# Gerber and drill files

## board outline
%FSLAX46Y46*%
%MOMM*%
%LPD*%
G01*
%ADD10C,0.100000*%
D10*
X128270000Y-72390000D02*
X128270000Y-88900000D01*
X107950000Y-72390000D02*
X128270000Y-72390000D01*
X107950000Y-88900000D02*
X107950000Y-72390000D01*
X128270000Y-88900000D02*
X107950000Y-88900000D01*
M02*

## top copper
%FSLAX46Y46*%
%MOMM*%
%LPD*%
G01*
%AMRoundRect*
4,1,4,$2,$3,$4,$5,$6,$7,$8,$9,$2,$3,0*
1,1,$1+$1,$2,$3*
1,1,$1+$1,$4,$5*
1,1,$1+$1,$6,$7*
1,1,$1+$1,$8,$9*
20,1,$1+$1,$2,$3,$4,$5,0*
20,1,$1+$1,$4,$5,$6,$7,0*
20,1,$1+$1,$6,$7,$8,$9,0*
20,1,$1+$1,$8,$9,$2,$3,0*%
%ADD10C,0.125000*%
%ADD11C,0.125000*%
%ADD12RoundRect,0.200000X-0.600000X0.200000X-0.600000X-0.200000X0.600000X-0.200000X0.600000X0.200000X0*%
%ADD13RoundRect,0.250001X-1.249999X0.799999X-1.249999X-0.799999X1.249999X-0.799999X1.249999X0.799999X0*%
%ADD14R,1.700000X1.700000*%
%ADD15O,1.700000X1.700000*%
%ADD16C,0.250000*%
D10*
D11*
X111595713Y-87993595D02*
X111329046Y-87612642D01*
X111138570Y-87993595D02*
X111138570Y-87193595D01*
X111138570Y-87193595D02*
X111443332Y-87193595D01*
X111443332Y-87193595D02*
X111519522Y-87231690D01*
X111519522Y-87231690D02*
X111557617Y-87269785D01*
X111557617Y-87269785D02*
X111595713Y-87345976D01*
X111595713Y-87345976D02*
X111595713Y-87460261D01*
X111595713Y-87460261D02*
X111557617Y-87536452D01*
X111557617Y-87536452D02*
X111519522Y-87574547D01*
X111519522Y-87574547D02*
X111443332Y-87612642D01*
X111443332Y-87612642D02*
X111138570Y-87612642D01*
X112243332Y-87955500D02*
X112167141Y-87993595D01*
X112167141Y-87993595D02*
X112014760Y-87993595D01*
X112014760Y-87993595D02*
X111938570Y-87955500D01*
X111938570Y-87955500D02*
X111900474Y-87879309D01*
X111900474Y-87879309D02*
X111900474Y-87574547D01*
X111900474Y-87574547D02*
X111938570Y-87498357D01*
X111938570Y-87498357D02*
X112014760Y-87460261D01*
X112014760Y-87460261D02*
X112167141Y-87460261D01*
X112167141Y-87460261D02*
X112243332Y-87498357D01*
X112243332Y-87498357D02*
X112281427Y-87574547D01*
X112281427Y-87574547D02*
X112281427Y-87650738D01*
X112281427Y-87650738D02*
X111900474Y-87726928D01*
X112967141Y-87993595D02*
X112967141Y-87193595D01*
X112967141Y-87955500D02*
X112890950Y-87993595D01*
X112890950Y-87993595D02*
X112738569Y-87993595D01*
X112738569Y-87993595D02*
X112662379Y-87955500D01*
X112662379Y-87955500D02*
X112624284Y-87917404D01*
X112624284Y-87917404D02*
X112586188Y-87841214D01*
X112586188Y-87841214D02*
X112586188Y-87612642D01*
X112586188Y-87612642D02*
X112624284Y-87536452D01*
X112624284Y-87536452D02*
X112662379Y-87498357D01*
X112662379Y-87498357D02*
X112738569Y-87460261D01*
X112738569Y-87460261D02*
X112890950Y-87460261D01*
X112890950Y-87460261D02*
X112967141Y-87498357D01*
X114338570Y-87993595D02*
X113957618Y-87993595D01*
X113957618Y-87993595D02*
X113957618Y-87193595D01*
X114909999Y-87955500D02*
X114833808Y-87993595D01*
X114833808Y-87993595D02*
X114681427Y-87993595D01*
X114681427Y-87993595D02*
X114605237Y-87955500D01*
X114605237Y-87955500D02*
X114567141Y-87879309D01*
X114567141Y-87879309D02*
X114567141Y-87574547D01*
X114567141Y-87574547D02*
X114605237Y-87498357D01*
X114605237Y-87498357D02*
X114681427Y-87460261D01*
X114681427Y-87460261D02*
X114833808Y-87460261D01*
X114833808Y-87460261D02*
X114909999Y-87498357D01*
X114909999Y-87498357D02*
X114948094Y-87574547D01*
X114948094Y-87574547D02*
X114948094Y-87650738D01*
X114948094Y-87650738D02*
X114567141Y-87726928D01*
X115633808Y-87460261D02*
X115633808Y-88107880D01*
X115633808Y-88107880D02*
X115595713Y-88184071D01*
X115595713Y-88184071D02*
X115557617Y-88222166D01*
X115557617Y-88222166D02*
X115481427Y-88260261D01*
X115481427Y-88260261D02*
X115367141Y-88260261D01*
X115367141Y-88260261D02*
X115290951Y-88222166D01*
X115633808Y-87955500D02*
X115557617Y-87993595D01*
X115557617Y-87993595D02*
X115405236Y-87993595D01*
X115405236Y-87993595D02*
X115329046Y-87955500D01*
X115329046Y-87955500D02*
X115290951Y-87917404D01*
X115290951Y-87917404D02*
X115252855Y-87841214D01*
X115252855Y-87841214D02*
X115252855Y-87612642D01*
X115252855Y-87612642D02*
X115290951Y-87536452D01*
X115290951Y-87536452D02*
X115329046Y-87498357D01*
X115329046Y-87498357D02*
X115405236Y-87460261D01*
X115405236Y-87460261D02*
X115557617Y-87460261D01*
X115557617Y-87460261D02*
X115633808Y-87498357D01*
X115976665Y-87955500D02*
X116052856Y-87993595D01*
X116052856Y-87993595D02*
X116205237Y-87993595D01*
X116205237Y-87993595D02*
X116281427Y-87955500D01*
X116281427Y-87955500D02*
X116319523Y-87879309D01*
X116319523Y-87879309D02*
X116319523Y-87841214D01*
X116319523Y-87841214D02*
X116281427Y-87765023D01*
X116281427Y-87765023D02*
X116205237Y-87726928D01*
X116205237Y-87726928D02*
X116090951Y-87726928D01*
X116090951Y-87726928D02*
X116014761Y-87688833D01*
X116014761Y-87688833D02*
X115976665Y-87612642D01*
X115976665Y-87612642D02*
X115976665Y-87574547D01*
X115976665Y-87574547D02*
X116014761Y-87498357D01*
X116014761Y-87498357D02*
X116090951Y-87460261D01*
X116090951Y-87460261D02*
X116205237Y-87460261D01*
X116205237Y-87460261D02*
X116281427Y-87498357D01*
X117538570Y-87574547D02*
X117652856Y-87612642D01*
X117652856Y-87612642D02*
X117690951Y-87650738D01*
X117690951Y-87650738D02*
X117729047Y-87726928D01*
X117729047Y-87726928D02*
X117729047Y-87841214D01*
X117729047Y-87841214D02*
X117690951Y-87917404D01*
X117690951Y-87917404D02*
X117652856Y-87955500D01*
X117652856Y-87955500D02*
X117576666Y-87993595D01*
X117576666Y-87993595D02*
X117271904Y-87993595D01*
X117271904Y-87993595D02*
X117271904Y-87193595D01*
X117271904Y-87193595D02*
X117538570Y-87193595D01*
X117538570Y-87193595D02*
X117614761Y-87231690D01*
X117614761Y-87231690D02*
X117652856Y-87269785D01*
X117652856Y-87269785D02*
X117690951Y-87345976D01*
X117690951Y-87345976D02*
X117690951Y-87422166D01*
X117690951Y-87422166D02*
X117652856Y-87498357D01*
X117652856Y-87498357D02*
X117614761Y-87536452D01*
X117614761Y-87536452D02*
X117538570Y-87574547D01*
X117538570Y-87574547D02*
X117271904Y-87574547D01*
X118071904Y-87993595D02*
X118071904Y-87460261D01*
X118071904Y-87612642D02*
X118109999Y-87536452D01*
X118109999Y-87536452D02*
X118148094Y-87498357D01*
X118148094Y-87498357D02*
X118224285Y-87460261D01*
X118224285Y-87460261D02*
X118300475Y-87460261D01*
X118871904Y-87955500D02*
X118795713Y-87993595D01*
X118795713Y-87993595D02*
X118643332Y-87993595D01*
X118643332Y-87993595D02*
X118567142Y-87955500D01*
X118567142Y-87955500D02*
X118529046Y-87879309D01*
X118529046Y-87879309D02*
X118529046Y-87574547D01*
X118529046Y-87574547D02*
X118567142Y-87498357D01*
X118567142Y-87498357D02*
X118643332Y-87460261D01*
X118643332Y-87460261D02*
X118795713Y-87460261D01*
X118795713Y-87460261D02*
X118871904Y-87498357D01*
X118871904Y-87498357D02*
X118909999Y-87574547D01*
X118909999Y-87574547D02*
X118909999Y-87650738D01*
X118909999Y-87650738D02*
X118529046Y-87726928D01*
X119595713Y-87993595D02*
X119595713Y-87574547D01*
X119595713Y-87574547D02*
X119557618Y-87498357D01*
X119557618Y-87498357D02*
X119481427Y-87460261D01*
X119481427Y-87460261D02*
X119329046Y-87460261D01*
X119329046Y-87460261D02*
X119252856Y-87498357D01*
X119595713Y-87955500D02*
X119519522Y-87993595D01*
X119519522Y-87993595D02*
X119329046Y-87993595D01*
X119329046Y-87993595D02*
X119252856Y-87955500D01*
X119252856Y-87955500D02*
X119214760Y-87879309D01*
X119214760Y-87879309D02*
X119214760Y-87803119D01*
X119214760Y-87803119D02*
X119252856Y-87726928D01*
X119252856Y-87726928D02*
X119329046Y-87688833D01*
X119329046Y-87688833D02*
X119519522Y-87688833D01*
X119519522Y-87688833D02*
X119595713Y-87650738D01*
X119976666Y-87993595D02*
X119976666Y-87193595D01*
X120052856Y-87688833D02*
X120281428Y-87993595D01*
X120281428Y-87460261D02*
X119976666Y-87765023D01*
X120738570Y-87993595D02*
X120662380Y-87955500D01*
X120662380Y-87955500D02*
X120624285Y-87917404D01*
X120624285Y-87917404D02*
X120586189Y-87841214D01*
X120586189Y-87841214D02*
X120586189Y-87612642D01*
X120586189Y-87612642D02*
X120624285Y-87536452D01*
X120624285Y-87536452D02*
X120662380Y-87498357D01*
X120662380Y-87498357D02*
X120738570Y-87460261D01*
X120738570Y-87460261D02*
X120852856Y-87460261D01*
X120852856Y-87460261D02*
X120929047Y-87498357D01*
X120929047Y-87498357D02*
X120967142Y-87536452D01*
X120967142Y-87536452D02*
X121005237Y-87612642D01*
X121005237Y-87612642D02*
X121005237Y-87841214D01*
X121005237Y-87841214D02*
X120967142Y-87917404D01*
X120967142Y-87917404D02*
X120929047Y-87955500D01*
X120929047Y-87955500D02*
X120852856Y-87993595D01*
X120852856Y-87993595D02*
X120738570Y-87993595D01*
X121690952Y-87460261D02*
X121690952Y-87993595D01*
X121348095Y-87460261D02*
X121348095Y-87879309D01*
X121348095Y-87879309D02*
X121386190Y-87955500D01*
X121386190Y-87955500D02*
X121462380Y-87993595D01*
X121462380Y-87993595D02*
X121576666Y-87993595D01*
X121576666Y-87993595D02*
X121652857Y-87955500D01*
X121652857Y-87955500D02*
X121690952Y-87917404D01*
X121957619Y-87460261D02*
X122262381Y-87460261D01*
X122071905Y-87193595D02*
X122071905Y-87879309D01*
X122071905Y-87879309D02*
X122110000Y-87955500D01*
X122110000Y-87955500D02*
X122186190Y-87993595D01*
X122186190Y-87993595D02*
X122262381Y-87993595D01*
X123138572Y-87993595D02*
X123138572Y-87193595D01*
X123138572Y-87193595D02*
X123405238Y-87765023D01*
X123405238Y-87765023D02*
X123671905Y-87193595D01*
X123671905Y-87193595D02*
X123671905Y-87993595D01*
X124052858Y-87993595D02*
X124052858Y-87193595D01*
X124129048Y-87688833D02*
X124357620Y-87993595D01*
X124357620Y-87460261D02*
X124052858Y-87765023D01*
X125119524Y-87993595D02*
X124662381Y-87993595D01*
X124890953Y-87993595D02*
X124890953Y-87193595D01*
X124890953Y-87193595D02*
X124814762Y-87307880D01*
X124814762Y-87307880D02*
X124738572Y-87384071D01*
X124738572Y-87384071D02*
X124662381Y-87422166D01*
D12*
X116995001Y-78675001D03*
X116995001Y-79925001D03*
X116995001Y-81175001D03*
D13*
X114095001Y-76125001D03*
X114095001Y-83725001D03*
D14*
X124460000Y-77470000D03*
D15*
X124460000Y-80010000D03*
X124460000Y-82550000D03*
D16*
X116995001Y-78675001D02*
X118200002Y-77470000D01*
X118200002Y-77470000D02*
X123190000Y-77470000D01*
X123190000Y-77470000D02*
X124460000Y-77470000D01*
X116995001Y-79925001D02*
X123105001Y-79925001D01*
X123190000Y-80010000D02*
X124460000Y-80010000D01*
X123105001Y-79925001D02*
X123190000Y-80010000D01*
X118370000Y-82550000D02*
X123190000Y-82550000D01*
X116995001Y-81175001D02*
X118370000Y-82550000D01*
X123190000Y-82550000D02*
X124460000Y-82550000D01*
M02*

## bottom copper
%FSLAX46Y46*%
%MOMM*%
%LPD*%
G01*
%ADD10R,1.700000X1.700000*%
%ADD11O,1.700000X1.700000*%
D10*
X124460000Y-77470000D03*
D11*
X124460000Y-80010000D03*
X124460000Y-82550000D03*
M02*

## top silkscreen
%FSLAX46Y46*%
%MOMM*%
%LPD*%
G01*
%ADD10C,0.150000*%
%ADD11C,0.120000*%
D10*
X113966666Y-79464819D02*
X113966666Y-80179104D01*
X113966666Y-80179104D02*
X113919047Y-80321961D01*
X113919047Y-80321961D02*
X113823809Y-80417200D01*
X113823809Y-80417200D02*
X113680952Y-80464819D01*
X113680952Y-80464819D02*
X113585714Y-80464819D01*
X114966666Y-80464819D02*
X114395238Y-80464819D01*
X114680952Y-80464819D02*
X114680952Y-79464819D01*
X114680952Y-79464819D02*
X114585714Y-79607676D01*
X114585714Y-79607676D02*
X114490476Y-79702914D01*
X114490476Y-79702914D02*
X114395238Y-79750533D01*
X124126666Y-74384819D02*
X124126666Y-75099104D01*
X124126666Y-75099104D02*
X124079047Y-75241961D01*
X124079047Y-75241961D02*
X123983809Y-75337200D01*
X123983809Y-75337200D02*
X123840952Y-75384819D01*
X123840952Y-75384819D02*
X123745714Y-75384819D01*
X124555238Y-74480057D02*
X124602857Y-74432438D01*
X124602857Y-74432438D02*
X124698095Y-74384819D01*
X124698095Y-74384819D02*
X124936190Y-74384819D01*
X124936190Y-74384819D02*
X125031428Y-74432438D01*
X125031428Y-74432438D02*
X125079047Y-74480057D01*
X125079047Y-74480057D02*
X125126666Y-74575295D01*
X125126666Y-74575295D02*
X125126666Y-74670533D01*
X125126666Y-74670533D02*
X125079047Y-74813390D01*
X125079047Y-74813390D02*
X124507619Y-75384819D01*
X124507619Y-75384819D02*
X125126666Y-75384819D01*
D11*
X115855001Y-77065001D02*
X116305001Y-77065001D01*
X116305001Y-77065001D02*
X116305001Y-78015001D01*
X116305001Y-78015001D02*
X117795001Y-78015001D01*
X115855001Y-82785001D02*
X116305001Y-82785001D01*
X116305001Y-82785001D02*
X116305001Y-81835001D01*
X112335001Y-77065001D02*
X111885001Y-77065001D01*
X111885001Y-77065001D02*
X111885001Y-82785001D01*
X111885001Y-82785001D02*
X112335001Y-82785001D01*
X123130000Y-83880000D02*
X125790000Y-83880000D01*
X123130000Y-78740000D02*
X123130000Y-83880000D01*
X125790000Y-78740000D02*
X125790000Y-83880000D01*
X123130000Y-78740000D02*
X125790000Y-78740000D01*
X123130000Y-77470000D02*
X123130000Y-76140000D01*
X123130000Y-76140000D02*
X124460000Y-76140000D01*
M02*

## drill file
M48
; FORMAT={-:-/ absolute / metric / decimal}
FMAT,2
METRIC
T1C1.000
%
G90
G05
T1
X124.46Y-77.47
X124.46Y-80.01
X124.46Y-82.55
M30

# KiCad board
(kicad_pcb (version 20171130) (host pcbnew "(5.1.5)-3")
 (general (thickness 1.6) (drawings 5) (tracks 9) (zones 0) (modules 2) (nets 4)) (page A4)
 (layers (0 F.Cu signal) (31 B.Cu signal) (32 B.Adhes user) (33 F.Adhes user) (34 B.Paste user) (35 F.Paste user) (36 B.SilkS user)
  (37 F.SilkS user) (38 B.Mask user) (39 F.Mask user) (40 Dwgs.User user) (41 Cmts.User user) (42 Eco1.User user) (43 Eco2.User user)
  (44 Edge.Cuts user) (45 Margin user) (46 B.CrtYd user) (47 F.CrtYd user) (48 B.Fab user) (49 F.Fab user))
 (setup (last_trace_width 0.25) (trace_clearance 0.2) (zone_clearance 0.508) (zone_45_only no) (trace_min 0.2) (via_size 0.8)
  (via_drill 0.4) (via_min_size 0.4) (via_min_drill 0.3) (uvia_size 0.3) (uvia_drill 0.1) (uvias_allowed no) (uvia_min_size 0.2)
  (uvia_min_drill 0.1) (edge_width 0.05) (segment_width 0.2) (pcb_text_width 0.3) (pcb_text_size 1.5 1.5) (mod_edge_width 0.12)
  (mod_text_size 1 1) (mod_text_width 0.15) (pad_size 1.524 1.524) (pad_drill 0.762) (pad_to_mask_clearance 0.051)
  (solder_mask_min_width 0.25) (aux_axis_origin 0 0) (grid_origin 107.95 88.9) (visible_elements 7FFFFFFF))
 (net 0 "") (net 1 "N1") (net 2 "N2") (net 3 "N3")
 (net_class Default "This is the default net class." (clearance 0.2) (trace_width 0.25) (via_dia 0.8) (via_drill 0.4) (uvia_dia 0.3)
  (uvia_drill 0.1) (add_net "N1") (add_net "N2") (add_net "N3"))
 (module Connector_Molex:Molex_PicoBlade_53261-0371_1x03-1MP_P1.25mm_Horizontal (layer F.Cu) (at 114.595001 79.925001 270)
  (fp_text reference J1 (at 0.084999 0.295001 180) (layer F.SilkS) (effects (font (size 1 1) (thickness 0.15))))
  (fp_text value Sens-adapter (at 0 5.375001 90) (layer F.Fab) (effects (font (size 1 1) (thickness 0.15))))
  (fp_line (start -2.86 -1.26) (end -2.86 -1.71) (layer F.SilkS) (width 0.12))
  (fp_line (start -2.86 -1.71) (end -1.91 -1.71) (layer F.SilkS) (width 0.12))
  (fp_line (start -1.91 -1.71) (end -1.91 -3.2) (layer F.SilkS) (width 0.12))
  (fp_line (start 2.86 -1.26) (end 2.86 -1.71) (layer F.SilkS) (width 0.12))
  (fp_line (start 2.86 -1.71) (end 1.91 -1.71) (layer F.SilkS) (width 0.12))
  (fp_line (start -2.86 2.26) (end -2.86 2.71) (layer F.SilkS) (width 0.12))
  (fp_line (start -2.86 2.71) (end 2.86 2.71) (layer F.SilkS) (width 0.12))
  (fp_line (start 2.86 2.71) (end 2.86 2.26) (layer F.SilkS) (width 0.12))
  (pad 1 smd roundrect (at -1.25 -2.4 270) (size 0.8 1.6) (layers F.Cu F.Paste F.Mask) (roundrect_rratio 0.25) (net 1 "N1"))
  (pad 2 smd roundrect (at 0 -2.4 270) (size 0.8 1.6) (layers F.Cu F.Paste F.Mask) (roundrect_rratio 0.25) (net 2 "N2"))
  (pad 3 smd roundrect (at 1.25 -2.4 270) (size 0.8 1.6) (layers F.Cu F.Paste F.Mask) (roundrect_rratio 0.25) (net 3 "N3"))
  (pad MP smd roundrect (at -3.8 0.5 270) (size 2.1 3) (layers F.Cu F.Paste F.Mask) (roundrect_rratio 0.119048))
  (pad MP smd roundrect (at 3.8 0.5 270) (size 2.1 3) (layers F.Cu F.Paste F.Mask) (roundrect_rratio 0.119048)))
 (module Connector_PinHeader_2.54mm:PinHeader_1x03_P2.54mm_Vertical (layer F.Cu) (at 124.46 77.47)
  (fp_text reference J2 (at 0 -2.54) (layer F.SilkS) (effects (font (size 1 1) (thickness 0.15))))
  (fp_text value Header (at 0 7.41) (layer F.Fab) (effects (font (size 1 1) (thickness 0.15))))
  (fp_line (start -1.33 6.41) (end 1.33 6.41) (layer F.SilkS) (width 0.12))
  (fp_line (start -1.33 1.27) (end -1.33 6.41) (layer F.SilkS) (width 0.12))
  (fp_line (start 1.33 1.27) (end 1.33 6.41) (layer F.SilkS) (width 0.12))
  (fp_line (start -1.33 1.27) (end 1.33 1.27) (layer F.SilkS) (width 0.12))
  (fp_line (start -1.33 0) (end -1.33 -1.33) (layer F.SilkS) (width 0.12))
  (fp_line (start -1.33 -1.33) (end 0 -1.33) (layer F.SilkS) (width 0.12))
  (pad 1 thru_hole rect (at 0 0) (size 1.7 1.7) (drill 1) (layers *.Cu *.Mask) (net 1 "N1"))
  (pad 2 thru_hole oval (at 0 2.54) (size 1.7 1.7) (drill 1) (layers *.Cu *.Mask) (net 2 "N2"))
  (pad 3 thru_hole oval (at 0 5.08) (size 1.7 1.7) (drill 1) (layers *.Cu *.Mask) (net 3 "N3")))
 (gr_line (start 128.27 72.39) (end 128.27 88.9) (layer Edge.Cuts) (width 0.1))
 (gr_line (start 107.95 72.39) (end 128.27 72.39) (layer Edge.Cuts) (width 0.1))
 (gr_line (start 107.95 88.9) (end 107.95 72.39) (layer Edge.Cuts) (width 0.1))
 (gr_line (start 128.27 88.9) (end 107.95 88.9) (layer Edge.Cuts) (width 0.1))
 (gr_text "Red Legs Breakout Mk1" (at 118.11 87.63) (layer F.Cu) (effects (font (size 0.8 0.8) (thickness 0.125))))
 (segment (start 116.995001 78.675001) (end 118.200002 77.47) (width 0.25) (layer F.Cu) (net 1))
 (segment (start 118.200002 77.47) (end 123.19 77.47) (width 0.25) (layer F.Cu) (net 1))
 (segment (start 123.19 77.47) (end 124.46 77.47) (width 0.25) (layer F.Cu) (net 1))
 (segment (start 116.995001 79.925001) (end 123.105001 79.925001) (width 0.25) (layer F.Cu) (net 2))
 (segment (start 123.19 80.01) (end 124.46 80.01) (width 0.25) (layer F.Cu) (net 2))
 (segment (start 123.105001 79.925001) (end 123.19 80.01) (width 0.25) (layer F.Cu) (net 2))
 (segment (start 118.37 82.55) (end 123.19 82.55) (width 0.25) (layer F.Cu) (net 3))
 (segment (start 116.995001 81.175001) (end 118.37 82.55) (width 0.25) (layer F.Cu) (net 3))
 (segment (start 123.19 82.55) (end 124.46 82.55) (width 0.25) (layer F.Cu) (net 3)))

